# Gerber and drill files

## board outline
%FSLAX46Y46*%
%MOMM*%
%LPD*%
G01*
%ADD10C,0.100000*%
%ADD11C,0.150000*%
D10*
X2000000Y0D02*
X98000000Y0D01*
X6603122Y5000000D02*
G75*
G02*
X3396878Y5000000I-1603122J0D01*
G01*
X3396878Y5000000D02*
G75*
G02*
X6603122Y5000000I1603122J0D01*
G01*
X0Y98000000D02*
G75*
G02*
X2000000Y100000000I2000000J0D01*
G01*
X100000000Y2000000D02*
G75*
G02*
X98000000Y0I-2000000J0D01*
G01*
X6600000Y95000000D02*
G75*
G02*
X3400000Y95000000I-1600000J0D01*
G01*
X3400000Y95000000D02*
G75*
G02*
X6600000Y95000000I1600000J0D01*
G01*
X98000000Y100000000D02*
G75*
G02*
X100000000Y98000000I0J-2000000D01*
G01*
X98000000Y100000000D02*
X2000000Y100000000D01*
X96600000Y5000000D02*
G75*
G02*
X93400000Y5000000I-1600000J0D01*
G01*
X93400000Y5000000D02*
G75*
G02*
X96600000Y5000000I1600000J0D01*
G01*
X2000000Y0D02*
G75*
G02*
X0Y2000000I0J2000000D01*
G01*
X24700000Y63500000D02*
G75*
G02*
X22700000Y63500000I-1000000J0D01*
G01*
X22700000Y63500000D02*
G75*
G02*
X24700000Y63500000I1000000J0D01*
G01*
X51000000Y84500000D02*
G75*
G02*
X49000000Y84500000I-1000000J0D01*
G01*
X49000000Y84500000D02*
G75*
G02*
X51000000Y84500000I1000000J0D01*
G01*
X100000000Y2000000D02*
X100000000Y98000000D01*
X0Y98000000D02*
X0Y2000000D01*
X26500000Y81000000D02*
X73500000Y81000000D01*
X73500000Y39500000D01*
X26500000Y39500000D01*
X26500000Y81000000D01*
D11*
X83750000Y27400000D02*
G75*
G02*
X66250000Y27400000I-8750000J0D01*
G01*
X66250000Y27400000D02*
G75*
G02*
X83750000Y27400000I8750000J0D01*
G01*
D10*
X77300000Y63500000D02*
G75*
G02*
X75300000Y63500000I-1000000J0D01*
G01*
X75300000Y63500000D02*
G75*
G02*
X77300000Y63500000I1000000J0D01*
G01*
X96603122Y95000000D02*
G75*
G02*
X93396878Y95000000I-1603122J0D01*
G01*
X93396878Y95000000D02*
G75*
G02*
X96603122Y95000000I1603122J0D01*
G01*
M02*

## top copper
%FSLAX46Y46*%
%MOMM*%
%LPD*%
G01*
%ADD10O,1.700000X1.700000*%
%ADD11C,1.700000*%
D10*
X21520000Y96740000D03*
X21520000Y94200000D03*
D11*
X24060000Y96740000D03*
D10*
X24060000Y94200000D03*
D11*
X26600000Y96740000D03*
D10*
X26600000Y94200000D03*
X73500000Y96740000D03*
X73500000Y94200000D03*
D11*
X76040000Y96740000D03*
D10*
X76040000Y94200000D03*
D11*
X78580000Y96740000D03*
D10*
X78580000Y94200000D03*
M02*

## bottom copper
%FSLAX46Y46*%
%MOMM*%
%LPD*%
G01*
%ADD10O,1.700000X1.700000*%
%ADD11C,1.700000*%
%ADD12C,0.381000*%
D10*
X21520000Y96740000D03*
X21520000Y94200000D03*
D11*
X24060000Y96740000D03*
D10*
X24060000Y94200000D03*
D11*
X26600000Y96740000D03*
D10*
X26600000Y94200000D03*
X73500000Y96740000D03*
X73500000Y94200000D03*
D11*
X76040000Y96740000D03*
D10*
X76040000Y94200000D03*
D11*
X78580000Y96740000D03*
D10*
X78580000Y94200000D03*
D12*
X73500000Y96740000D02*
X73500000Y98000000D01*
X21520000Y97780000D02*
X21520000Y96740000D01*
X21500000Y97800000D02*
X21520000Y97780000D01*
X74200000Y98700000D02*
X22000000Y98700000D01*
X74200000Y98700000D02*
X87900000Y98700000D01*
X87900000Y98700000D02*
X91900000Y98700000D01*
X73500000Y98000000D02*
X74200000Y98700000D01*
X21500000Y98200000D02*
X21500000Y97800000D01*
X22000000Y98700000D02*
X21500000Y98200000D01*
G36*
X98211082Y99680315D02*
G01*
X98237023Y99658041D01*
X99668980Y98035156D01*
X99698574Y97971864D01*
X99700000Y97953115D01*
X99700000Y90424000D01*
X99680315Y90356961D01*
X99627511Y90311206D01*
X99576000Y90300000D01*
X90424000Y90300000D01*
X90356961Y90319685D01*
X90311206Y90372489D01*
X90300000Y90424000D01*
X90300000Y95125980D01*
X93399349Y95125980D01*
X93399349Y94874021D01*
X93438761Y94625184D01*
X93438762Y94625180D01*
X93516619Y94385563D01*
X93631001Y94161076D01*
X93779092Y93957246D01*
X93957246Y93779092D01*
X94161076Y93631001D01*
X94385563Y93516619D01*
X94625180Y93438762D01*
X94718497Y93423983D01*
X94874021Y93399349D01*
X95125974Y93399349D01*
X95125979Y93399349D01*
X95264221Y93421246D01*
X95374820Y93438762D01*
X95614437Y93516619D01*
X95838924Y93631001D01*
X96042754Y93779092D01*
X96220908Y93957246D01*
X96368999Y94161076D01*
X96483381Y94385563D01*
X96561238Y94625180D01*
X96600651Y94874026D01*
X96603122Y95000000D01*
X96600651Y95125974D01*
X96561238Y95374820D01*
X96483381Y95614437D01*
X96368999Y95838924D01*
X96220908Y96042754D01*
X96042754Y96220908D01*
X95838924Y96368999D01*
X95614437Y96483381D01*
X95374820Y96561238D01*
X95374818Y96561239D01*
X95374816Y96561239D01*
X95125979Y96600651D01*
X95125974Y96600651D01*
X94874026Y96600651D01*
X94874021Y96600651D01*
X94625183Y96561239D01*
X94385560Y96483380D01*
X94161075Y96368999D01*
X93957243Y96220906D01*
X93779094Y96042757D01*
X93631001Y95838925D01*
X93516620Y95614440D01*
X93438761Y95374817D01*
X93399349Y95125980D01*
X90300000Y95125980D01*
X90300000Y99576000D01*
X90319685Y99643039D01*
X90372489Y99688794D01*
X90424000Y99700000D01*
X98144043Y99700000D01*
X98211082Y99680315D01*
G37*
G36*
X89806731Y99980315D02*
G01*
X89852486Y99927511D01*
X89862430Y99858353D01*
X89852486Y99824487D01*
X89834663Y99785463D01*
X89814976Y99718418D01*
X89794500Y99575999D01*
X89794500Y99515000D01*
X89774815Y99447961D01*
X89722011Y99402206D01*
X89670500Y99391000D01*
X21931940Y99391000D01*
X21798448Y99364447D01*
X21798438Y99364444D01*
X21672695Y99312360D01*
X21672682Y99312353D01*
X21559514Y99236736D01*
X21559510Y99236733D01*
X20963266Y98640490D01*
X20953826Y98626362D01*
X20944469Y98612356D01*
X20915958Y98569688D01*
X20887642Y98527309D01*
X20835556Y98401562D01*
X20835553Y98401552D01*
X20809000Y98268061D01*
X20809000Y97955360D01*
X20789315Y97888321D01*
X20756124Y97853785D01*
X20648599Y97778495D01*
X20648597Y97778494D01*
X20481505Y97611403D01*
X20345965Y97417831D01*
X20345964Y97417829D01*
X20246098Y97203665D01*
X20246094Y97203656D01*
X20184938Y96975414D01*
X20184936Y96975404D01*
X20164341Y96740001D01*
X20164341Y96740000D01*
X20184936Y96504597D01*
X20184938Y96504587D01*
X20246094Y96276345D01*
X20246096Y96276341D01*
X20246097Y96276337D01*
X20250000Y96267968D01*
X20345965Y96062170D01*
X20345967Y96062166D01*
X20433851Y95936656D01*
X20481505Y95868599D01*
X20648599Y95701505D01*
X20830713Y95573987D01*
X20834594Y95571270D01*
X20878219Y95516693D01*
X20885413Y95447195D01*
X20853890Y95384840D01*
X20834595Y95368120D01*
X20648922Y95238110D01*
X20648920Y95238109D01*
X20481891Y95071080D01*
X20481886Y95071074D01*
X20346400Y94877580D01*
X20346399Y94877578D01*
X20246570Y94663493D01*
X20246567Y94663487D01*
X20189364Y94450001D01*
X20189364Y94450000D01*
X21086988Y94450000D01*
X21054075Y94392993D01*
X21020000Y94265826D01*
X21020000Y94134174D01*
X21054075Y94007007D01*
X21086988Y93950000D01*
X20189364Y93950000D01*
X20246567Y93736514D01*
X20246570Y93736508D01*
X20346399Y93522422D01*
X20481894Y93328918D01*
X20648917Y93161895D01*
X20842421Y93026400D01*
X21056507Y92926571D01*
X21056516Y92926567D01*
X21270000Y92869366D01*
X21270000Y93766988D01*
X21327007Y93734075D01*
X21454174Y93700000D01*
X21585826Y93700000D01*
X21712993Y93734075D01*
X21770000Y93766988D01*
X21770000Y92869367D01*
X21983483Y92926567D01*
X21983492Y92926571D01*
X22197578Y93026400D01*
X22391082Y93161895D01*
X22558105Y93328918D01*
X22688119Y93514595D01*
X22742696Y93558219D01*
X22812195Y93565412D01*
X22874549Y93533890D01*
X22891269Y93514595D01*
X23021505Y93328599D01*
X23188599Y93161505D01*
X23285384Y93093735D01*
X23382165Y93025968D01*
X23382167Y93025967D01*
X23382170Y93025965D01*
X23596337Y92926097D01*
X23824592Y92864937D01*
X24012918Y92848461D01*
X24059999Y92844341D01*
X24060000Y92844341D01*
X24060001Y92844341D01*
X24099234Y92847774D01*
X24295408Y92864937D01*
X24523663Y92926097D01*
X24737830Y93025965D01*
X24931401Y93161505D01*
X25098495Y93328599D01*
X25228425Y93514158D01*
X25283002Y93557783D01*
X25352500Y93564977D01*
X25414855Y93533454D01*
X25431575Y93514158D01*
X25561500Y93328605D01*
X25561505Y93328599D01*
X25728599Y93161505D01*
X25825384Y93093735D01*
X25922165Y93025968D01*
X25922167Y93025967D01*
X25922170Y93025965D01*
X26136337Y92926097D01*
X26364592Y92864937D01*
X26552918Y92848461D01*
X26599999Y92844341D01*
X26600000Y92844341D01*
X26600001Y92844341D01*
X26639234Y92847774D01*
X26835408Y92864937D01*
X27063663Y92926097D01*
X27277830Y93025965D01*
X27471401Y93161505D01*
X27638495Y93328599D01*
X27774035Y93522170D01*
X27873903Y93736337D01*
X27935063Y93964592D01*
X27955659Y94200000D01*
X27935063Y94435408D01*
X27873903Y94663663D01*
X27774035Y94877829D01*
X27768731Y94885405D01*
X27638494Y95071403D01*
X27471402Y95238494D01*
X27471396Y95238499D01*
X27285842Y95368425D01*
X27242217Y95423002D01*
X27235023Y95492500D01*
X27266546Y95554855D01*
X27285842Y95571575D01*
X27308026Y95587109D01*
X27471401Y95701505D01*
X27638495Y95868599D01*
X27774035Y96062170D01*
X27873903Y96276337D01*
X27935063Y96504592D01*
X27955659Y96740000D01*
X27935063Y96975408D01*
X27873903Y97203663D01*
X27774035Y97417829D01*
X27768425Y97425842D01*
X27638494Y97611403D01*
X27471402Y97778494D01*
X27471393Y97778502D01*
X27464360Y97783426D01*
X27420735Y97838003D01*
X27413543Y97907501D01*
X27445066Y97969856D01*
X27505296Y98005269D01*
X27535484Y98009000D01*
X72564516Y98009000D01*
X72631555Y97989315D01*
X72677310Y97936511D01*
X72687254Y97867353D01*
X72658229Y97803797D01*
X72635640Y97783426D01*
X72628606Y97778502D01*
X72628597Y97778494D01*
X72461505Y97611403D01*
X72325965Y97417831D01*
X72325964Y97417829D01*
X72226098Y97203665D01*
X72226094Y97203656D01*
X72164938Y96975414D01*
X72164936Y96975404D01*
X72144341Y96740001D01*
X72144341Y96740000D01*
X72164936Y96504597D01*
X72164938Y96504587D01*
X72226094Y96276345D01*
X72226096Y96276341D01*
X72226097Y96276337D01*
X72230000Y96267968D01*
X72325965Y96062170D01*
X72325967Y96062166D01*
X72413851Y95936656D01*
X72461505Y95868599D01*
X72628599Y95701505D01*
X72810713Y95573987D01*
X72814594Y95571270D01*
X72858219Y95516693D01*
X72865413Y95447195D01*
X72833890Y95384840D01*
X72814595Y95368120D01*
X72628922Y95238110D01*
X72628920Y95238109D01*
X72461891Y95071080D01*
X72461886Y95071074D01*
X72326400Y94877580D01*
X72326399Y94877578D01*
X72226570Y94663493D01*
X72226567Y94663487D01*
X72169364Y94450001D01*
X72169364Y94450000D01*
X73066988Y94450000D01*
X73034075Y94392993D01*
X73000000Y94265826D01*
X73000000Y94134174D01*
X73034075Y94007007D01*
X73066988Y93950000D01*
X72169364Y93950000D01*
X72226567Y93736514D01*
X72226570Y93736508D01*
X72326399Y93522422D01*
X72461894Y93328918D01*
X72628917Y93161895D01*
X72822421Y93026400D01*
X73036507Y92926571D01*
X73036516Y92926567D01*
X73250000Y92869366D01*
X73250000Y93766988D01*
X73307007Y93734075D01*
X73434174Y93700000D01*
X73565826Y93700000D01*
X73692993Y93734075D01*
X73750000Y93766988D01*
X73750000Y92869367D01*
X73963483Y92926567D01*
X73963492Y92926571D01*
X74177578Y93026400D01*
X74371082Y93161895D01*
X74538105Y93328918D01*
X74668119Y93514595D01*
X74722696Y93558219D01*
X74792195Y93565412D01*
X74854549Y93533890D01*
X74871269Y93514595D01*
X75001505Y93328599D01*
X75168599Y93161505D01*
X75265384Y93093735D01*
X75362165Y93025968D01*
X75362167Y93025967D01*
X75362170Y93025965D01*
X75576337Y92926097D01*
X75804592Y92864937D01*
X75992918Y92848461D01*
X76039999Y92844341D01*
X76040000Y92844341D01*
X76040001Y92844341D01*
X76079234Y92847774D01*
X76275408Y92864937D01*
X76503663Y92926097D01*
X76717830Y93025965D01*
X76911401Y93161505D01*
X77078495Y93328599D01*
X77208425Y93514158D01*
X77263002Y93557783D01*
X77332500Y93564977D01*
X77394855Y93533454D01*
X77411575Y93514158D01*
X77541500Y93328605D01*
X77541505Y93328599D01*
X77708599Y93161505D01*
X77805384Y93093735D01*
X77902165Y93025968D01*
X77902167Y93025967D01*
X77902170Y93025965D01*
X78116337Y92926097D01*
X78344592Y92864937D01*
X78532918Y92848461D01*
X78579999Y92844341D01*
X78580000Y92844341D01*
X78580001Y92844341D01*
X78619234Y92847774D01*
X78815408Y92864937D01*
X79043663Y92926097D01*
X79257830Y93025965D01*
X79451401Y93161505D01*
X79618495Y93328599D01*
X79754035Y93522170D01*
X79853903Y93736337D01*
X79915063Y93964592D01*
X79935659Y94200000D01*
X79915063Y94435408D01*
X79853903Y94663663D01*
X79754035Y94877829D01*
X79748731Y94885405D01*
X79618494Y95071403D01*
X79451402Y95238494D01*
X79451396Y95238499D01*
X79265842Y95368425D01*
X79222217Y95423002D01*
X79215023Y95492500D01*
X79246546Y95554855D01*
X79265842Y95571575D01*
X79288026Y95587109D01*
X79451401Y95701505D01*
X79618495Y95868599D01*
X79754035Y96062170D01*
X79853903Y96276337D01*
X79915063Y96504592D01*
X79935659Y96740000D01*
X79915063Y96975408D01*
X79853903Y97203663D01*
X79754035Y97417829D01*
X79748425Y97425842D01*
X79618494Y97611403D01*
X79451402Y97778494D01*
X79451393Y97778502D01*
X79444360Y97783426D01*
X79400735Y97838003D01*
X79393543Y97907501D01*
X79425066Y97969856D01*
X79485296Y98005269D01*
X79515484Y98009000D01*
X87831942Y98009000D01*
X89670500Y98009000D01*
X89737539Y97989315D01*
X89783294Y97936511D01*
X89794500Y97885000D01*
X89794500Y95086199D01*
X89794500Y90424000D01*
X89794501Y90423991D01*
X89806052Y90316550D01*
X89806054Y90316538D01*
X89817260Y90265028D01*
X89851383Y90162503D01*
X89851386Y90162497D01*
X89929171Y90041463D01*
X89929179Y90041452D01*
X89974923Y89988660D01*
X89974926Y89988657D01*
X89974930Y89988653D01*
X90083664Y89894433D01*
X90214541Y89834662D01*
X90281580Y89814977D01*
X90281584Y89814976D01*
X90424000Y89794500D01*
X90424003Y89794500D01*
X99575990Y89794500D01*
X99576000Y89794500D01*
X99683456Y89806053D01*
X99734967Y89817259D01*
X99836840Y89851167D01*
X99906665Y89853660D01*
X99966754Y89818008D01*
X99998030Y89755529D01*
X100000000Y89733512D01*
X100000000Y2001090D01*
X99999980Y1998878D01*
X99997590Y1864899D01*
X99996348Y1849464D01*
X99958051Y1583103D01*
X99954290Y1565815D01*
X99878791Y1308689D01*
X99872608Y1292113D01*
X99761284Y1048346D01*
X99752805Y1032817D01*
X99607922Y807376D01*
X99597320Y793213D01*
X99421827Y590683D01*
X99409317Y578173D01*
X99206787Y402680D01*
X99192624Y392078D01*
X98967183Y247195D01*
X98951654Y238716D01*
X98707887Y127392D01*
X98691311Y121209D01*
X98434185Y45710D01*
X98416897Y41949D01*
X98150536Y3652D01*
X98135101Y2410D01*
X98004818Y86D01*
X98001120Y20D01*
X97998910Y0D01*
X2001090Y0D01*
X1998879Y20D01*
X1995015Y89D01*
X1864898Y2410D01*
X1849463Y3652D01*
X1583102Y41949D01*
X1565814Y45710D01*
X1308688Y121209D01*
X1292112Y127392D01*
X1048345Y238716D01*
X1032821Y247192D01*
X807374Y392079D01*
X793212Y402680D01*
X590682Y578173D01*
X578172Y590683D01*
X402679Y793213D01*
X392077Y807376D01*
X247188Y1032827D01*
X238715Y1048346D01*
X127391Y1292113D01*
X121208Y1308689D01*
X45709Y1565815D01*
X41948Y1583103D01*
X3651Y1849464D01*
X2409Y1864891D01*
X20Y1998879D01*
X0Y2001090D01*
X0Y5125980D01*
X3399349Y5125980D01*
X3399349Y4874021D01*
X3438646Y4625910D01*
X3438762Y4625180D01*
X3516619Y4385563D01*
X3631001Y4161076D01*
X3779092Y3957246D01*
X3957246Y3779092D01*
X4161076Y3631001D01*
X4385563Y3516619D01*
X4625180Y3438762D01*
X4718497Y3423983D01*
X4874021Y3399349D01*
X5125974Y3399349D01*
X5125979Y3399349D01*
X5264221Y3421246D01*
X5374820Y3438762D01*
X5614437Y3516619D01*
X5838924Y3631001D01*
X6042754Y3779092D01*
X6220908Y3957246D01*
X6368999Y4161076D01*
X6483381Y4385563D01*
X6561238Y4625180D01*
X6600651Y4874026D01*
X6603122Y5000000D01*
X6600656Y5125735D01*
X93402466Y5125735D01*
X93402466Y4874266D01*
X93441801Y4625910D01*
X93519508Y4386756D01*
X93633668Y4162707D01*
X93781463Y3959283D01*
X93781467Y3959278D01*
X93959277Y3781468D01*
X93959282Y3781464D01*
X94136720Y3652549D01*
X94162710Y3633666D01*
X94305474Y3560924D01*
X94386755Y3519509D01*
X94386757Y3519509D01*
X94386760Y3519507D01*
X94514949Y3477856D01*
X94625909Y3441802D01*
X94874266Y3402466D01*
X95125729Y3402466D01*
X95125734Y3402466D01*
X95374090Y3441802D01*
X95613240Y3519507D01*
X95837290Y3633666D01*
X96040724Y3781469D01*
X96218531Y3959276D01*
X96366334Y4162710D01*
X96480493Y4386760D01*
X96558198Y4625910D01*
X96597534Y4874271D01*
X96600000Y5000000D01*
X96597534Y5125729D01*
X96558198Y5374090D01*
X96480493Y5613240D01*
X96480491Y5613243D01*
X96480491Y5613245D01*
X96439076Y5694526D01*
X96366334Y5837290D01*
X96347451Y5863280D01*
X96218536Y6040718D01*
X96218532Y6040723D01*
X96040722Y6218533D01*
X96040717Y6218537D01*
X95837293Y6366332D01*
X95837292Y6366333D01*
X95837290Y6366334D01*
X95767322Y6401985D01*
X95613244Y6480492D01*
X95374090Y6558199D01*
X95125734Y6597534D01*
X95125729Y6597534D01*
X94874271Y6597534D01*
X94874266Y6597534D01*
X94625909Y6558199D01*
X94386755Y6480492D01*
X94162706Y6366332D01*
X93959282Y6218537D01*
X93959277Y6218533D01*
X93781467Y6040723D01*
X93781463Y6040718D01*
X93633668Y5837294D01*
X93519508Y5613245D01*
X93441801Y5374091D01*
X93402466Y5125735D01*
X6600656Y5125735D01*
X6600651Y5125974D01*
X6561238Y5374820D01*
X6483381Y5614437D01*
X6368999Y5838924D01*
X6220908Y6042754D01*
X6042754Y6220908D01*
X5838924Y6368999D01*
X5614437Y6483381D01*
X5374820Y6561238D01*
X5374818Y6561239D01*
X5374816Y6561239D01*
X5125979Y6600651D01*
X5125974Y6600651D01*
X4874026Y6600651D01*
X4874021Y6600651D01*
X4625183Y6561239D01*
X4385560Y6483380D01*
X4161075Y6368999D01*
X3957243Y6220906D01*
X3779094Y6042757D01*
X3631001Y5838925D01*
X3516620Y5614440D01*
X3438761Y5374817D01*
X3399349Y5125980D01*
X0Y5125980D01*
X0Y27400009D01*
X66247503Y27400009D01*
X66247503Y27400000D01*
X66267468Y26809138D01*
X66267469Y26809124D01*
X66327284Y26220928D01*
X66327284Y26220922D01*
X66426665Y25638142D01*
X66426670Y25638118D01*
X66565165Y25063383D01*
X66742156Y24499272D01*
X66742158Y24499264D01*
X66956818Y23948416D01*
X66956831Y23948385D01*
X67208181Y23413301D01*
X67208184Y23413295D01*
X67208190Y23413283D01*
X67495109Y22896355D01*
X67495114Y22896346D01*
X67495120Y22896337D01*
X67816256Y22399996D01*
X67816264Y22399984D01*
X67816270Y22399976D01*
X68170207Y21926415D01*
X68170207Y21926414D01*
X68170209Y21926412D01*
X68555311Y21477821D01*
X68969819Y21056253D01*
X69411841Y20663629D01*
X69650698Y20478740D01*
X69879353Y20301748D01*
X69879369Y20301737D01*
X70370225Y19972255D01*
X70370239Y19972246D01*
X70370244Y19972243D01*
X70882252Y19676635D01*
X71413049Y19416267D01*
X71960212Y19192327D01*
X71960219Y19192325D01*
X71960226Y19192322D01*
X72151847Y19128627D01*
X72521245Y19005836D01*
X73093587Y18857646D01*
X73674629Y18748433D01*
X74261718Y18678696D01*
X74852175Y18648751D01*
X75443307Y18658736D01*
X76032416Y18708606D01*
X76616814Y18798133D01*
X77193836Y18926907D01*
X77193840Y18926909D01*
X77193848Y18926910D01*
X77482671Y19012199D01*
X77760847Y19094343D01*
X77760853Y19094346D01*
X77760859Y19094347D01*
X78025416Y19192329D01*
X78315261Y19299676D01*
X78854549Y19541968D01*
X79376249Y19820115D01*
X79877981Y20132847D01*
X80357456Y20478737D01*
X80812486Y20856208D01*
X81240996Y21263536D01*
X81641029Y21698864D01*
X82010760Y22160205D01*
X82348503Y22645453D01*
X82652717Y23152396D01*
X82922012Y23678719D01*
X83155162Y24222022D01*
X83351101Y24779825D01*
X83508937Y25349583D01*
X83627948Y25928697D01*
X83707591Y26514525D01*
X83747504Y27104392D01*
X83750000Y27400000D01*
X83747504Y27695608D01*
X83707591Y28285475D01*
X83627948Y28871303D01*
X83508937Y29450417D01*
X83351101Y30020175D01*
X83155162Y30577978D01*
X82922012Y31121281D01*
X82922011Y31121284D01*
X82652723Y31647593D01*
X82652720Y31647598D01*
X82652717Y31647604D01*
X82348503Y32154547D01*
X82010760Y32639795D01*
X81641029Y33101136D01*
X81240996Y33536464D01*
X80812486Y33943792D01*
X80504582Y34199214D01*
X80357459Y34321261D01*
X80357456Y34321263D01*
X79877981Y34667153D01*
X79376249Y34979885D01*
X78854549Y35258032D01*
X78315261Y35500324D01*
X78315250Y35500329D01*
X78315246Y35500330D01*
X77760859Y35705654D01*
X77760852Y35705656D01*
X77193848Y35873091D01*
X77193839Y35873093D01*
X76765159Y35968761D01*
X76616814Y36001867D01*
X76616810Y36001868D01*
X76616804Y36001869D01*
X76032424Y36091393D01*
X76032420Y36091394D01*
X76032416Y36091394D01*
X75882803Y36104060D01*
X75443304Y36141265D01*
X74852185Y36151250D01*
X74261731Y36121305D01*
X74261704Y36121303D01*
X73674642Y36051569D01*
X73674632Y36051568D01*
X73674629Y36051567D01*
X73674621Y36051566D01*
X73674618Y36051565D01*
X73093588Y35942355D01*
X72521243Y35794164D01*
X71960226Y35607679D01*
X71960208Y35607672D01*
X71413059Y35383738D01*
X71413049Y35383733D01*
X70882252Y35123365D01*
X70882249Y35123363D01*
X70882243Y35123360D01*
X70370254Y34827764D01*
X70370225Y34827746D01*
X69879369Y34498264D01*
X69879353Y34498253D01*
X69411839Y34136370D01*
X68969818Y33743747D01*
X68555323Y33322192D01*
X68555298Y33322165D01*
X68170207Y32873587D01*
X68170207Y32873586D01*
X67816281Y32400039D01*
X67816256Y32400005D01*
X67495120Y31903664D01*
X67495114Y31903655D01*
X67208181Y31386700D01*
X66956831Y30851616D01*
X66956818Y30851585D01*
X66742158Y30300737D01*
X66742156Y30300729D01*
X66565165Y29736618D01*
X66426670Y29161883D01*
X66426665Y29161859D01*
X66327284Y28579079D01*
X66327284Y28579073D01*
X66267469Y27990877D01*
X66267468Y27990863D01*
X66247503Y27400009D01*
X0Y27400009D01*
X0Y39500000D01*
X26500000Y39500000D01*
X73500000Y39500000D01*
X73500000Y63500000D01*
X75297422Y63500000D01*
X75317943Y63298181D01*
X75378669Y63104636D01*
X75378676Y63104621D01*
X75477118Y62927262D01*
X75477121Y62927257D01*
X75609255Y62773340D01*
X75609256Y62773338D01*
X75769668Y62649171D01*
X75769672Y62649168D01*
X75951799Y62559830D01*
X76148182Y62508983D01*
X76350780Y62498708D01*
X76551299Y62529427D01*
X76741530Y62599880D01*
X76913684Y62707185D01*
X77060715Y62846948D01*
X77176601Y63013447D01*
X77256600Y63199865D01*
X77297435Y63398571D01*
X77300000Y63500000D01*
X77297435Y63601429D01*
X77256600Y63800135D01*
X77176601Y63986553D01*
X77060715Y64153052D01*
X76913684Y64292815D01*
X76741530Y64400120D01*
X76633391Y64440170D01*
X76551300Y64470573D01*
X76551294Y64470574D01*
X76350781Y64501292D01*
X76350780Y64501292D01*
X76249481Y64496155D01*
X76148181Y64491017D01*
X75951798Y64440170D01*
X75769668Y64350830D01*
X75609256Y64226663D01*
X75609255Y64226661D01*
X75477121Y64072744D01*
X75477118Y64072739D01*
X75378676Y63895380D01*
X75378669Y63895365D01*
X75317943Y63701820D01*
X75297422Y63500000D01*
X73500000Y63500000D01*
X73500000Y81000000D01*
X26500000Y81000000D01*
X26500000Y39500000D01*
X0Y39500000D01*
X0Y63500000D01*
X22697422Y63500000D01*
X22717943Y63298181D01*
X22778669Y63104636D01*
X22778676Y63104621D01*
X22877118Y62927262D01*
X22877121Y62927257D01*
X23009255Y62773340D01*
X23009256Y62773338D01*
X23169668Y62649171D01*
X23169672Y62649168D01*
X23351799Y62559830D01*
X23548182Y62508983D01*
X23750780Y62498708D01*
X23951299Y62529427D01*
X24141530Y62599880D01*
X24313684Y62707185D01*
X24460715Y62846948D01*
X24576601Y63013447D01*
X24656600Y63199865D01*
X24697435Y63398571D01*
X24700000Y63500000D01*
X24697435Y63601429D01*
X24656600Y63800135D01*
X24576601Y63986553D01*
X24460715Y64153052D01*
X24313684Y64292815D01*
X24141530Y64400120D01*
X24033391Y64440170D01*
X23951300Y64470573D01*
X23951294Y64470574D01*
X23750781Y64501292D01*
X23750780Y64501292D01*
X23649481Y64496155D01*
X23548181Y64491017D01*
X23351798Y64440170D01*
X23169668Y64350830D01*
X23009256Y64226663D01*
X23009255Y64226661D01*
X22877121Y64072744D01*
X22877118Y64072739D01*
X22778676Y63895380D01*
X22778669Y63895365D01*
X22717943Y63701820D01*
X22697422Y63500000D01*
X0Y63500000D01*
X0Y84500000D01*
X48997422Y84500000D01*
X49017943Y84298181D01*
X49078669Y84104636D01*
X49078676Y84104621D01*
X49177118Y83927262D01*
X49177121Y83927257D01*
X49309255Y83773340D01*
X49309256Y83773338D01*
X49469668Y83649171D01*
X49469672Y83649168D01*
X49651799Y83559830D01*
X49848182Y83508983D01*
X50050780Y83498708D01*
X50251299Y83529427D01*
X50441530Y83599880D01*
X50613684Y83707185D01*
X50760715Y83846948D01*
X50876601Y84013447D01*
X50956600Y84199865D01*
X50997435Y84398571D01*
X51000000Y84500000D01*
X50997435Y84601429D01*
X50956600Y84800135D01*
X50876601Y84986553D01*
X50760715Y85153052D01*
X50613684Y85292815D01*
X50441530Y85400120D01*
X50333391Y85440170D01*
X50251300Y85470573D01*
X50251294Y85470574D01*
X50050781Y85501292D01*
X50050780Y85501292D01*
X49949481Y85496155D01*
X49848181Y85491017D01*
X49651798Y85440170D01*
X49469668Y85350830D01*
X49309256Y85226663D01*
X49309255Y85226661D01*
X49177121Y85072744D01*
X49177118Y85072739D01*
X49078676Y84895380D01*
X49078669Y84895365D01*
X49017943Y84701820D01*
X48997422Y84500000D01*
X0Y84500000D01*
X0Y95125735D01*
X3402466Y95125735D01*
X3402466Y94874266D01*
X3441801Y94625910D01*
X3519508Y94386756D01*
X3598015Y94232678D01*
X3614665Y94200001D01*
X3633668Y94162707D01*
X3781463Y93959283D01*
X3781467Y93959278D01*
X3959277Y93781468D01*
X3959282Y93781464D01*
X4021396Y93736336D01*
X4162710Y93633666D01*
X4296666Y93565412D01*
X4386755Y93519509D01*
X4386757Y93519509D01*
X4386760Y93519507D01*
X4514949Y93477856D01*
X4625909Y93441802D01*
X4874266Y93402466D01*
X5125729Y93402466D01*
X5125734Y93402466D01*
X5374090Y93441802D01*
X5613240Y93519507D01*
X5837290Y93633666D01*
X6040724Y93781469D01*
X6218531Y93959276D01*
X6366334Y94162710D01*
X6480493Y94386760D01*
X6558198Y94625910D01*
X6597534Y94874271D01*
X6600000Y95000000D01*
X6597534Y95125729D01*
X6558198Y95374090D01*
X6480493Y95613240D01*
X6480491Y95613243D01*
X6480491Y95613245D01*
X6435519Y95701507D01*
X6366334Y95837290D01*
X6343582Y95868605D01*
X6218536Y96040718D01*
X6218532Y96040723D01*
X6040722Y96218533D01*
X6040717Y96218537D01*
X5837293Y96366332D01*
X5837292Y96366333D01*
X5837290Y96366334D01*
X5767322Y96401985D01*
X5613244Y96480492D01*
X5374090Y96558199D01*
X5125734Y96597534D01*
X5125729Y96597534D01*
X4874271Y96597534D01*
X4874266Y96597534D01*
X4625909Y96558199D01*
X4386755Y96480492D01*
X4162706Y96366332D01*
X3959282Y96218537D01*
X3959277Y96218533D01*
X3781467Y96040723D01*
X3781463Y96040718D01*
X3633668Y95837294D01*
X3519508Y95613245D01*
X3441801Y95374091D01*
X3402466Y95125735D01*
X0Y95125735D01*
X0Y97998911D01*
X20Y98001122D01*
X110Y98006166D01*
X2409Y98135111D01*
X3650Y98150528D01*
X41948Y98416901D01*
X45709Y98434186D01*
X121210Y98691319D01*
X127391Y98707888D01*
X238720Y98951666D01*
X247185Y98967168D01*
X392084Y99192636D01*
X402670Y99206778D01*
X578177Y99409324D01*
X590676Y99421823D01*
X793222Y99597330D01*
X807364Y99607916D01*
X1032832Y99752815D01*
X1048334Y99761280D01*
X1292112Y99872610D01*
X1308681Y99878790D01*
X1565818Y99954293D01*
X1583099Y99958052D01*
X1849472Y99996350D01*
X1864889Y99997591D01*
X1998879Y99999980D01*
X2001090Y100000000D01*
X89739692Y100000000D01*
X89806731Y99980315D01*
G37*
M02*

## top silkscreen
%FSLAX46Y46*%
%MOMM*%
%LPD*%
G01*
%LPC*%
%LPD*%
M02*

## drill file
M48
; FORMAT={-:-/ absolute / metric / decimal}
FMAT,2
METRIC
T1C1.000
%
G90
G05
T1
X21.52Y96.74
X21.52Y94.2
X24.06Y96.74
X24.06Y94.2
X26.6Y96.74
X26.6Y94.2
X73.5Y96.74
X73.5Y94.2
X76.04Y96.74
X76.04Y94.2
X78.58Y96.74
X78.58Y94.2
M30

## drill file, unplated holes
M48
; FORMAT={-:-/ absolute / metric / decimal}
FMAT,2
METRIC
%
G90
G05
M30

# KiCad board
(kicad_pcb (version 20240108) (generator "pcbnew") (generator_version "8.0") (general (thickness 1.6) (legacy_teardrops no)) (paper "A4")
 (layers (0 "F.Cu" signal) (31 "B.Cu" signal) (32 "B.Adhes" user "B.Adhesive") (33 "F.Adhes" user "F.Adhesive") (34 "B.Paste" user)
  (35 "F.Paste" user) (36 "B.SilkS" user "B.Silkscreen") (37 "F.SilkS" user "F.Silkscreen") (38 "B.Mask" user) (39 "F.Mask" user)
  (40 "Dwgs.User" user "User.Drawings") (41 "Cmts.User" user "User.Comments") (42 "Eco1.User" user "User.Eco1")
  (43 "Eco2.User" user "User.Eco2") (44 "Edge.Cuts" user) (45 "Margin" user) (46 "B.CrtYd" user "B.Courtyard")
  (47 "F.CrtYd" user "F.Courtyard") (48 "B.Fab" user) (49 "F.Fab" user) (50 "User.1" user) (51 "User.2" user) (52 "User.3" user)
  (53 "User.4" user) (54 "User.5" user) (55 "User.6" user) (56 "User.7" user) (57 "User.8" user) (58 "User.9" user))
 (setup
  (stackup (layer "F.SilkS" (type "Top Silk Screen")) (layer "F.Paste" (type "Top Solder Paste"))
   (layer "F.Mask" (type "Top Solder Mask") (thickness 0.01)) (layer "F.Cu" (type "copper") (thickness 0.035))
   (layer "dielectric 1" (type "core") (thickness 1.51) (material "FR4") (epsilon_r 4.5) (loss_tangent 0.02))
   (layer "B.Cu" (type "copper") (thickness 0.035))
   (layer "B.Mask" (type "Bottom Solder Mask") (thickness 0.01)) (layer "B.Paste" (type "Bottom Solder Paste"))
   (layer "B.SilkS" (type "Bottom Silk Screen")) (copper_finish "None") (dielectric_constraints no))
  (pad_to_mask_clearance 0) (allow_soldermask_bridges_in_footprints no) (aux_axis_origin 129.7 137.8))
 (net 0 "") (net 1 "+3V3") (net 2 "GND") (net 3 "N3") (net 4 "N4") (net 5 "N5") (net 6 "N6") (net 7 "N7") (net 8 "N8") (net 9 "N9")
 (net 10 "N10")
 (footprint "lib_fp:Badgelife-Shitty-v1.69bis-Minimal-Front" (layer "F.Cu") (at 153.76 42.33)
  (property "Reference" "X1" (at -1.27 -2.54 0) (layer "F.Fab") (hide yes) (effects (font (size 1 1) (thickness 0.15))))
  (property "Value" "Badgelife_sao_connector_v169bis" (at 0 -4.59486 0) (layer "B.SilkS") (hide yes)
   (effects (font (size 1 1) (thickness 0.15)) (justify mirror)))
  (pad "1" thru_hole oval (at -2.54 -1.27) (size 1.7 1.7) (drill 1) (layers "*.Cu" "B.Mask") (remove_unused_layers no) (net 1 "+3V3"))
  (pad "2" thru_hole oval (at -2.54 1.27) (size 1.7 1.7) (drill 1) (layers "*.Cu" "B.Mask") (remove_unused_layers no) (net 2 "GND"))
  (pad "3" thru_hole circle (at 0 -1.27) (size 1.7 1.7) (drill 1) (layers "*.Cu" "B.Mask") (remove_unused_layers no) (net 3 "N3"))
  (pad "4" thru_hole oval (at 0 1.27) (size 1.7 1.7) (drill 1) (layers "*.Cu" "B.Mask") (remove_unused_layers no) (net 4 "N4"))
  (pad "5" thru_hole circle (at 2.54 -1.27) (size 1.7 1.7) (drill 1) (layers "*.Cu" "B.Mask") (remove_unused_layers no) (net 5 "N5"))
  (pad "6" thru_hole oval (at 2.54 1.27) (size 1.7 1.7) (drill 1) (layers "*.Cu" "B.Mask") (remove_unused_layers no) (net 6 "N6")))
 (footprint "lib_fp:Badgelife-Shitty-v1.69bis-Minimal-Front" (layer "F.Cu") (at 205.74 42.33)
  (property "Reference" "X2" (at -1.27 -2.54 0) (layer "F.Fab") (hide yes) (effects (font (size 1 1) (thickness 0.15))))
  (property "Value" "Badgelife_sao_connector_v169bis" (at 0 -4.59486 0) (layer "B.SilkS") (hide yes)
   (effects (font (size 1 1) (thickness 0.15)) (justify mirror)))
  (pad "1" thru_hole oval (at -2.54 -1.27) (size 1.7 1.7) (drill 1) (layers "*.Cu" "B.Mask") (remove_unused_layers no) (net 1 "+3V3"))
  (pad "2" thru_hole oval (at -2.54 1.27) (size 1.7 1.7) (drill 1) (layers "*.Cu" "B.Mask") (remove_unused_layers no) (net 2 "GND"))
  (pad "3" thru_hole circle (at 0 -1.27) (size 1.7 1.7) (drill 1) (layers "*.Cu" "B.Mask") (remove_unused_layers no) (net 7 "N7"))
  (pad "4" thru_hole oval (at 0 1.27) (size 1.7 1.7) (drill 1) (layers "*.Cu" "B.Mask") (remove_unused_layers no) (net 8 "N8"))
  (pad "5" thru_hole circle (at 2.54 -1.27) (size 1.7 1.7) (drill 1) (layers "*.Cu" "B.Mask") (remove_unused_layers no) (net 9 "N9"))
  (pad "6" thru_hole oval (at 2.54 1.27) (size 1.7 1.7) (drill 1) (layers "*.Cu" "B.Mask") (remove_unused_layers no) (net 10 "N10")))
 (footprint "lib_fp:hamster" (layer "B.Cu") (at 135.1 118.3 180)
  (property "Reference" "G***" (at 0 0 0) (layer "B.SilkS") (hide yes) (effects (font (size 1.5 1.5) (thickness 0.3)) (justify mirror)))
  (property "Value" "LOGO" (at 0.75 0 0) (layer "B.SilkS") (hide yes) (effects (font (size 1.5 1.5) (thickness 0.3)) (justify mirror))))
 (gr_line (start 131.7 137.8) (end 227.7 137.8) (stroke (width 0.1) (type default)) (layer "Edge.Cuts"))
 (gr_circle (center 134.7 132.8) (end 136.3 132.9) (stroke (width 0.1) (type default)) (fill none) (layer "Edge.Cuts"))
 (gr_arc (start 129.7 39.8) (mid 130.285786 38.385786) (end 131.7 37.8) (stroke (width 0.1) (type default)) (layer "Edge.Cuts"))
 (gr_arc (start 229.7 135.8) (mid 229.114214 137.214214) (end 227.7 137.8) (stroke (width 0.1) (type default)) (layer "Edge.Cuts"))
 (gr_circle (center 134.7 42.8) (end 136.3 42.8) (stroke (width 0.1) (type default)) (fill none) (layer "Edge.Cuts"))
 (gr_arc (start 227.7 37.8) (mid 229.114214 38.385786) (end 229.7 39.8) (stroke (width 0.1) (type default)) (layer "Edge.Cuts"))
 (gr_line (start 227.7 37.8) (end 131.7 37.8) (stroke (width 0.1) (type default)) (layer "Edge.Cuts"))
 (gr_circle (center 224.7 132.8) (end 226.3 132.8) (stroke (width 0.1) (type default)) (fill none) (layer "Edge.Cuts"))
 (gr_arc (start 131.7 137.8) (mid 130.285786 137.214214) (end 129.7 135.8) (stroke (width 0.1) (type default)) (layer "Edge.Cuts"))
 (gr_circle (center 153.4 74.3) (end 154.4 74.3) (stroke (width 0.1) (type default)) (fill none) (layer "Edge.Cuts"))
 (gr_circle (center 179.7 53.3) (end 180.7 53.3) (stroke (width 0.1) (type default)) (fill none) (layer "Edge.Cuts"))
 (gr_line (start 229.7 135.8) (end 229.7 39.8) (stroke (width 0.1) (type default)) (layer "Edge.Cuts"))
 (gr_line (start 129.7 39.8) (end 129.7 135.8) (stroke (width 0.1) (type default)) (layer "Edge.Cuts"))
 (gr_rect (start 156.2 56.8) (end 203.2 98.3) (stroke (width 0.1) (type default)) (fill none) (layer "Edge.Cuts"))
 (gr_circle (center 204.7 110.4) (end 213.45 110.4) (stroke (width 0.15) (type default)) (fill none) (layer "Edge.Cuts"))
 (gr_circle (center 206 74.3) (end 207 74.3) (stroke (width 0.1) (type default)) (fill none) (layer "Edge.Cuts"))
 (gr_circle (center 224.7 42.8) (end 226.3 42.9) (stroke (width 0.1) (type default)) (fill none) (layer "Edge.Cuts"))
 (segment (start 203.2 41.06) (end 203.2 39.8) (width 0.381) (layer "B.Cu") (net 1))
 (segment (start 151.22 40.02) (end 151.22 41.06) (width 0.381) (layer "B.Cu") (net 1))
 (segment (start 151.2 40) (end 151.22 40.02) (width 0.381) (layer "B.Cu") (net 1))
 (segment (start 203.9 39.1) (end 151.7 39.1) (width 0.381) (layer "B.Cu") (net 1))
 (segment (start 203.9 39.1) (end 217.6 39.1) (width 0.381) (layer "B.Cu") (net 1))
 (segment (start 217.6 39.1) (end 221.6 39.1) (width 0.381) (layer "B.Cu") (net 1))
 (segment (start 203.2 39.8) (end 203.9 39.1) (width 0.381) (layer "B.Cu") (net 1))
 (segment (start 151.2 39.6) (end 151.2 40) (width 0.381) (layer "B.Cu") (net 1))
 (segment (start 151.7 39.1) (end 151.2 39.6) (width 0.381) (layer "B.Cu") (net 1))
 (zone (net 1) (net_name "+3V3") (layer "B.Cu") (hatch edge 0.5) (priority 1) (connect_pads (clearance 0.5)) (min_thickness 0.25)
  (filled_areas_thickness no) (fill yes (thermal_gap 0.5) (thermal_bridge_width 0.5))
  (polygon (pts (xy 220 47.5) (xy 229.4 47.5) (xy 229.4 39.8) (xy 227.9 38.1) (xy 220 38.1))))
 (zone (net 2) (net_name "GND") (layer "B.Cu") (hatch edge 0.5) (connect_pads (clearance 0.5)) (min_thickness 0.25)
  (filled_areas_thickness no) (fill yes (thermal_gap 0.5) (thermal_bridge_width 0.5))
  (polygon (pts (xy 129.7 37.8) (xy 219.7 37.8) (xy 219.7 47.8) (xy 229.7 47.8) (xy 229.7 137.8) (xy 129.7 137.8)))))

